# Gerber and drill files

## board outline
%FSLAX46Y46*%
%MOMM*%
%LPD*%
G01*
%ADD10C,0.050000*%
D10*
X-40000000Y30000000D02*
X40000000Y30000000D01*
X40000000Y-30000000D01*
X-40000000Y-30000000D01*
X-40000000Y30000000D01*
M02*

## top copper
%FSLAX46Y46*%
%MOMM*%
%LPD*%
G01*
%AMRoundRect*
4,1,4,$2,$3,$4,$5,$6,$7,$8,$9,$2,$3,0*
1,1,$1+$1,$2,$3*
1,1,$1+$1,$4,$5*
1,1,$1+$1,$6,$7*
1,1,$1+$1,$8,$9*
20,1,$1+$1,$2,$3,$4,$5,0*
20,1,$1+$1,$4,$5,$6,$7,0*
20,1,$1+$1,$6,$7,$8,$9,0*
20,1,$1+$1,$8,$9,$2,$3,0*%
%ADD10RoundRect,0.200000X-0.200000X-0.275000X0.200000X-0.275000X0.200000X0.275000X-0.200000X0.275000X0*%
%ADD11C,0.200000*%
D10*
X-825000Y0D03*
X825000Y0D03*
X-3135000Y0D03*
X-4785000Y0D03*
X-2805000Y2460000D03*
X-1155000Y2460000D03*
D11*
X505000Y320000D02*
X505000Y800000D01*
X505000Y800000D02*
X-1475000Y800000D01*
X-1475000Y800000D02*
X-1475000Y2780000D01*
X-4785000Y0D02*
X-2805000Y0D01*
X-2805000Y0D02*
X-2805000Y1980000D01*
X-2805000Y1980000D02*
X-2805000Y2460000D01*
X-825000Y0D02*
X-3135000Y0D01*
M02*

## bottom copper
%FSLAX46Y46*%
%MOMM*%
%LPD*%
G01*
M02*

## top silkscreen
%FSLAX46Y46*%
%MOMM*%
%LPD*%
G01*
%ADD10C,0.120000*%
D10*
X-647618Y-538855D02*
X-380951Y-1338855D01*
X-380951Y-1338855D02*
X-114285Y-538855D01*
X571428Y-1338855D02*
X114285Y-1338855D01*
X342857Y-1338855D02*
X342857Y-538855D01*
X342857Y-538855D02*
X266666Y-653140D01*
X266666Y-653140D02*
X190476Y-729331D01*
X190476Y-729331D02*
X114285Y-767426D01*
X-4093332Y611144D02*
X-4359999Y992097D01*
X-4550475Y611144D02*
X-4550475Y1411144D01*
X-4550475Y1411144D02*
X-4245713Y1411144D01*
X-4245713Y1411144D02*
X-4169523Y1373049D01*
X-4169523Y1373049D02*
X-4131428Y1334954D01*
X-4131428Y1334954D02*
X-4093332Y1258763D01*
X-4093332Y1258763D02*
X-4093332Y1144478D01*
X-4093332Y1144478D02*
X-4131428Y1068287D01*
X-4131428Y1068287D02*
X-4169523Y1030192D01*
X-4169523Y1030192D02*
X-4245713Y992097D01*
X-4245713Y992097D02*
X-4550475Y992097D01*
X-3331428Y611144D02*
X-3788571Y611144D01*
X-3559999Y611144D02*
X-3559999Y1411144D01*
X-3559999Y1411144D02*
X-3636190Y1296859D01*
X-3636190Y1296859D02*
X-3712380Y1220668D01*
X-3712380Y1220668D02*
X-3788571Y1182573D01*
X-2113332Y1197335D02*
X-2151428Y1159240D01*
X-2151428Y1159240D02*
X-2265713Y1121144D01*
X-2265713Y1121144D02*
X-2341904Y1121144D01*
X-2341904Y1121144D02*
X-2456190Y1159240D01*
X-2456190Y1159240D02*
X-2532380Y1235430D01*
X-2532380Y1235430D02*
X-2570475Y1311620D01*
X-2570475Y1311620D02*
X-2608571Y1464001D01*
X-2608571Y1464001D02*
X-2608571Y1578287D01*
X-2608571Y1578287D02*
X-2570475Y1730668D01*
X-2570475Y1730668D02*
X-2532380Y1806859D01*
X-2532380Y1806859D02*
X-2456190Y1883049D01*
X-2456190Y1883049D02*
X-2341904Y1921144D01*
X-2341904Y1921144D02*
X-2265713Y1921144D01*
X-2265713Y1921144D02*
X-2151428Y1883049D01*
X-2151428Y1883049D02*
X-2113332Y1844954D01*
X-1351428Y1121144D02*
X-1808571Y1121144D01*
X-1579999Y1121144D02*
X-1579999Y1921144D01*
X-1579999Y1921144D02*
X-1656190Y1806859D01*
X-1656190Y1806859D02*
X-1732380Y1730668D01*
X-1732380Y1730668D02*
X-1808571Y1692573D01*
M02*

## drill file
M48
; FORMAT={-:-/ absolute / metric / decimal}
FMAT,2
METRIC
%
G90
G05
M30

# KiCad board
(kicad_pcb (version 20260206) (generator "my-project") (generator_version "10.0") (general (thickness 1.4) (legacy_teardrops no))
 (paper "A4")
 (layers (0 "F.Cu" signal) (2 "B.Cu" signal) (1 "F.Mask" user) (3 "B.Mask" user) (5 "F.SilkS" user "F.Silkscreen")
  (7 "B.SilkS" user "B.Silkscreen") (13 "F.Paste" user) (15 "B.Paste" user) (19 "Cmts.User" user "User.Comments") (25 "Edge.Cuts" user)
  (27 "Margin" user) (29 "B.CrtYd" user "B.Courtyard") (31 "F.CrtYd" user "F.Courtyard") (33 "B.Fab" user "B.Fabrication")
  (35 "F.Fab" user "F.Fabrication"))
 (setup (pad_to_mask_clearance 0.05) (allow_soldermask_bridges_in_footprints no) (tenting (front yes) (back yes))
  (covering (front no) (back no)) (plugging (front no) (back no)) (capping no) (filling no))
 (gr_rect (start -40.0000 -30.0000) (end 40.0000 30.0000) (stroke (width 0.05) (type solid)) (fill none) (layer "Edge.Cuts"))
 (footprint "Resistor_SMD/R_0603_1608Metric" (layer "F.Cu") (at 0.0000 0.0000 0)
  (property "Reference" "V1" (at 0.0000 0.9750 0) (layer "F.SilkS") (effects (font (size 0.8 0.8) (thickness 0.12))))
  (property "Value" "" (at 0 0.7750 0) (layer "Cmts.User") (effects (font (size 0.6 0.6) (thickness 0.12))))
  (pad 1 smd roundrect (at -0.8250 0.0000) (size 0.8000 0.9500) (layers "F.Cu" "F.Mask") (roundrect_rratio 0.25) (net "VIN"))
  (pad 2 smd roundrect (at 0.8250 0.0000) (size 0.8000 0.9500) (layers "F.Cu" "F.Mask") (roundrect_rratio 0.25) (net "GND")))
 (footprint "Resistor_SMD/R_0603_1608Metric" (layer "F.Cu") (at -3.9600 0.0000 180)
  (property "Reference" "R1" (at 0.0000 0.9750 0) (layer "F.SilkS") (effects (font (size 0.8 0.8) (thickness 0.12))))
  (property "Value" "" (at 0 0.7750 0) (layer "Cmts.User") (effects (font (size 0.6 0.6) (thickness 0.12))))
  (pad 1 smd roundrect (at -0.8250 0.0000) (size 0.8000 0.9500) (layers "F.Cu" "F.Mask") (roundrect_rratio 0.25) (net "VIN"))
  (pad 2 smd roundrect (at 0.8250 -0.0000) (size 0.8000 0.9500) (layers "F.Cu" "F.Mask") (roundrect_rratio 0.25) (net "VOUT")))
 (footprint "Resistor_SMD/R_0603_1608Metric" (layer "F.Cu") (at -1.9800 -2.4600 0)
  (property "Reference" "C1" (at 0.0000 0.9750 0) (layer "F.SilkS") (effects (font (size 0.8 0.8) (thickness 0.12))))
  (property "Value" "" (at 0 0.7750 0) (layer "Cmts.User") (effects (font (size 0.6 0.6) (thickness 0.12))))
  (pad 1 smd roundrect (at -0.8250 0.0000) (size 0.8000 0.9500) (layers "F.Cu" "F.Mask") (roundrect_rratio 0.25) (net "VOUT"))
  (pad 2 smd roundrect (at 0.8250 0.0000) (size 0.8000 0.9500) (layers "F.Cu" "F.Mask") (roundrect_rratio 0.25) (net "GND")))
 (segment (start 0.5050 -0.3200) (end 0.5050 -0.8000) (width 0.2) (layer "F.Cu") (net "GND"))
 (segment (start 0.5050 -0.8000) (end -1.4750 -0.8000) (width 0.2) (layer "F.Cu") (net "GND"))
 (segment (start -1.4750 -0.8000) (end -1.4750 -2.7800) (width 0.2) (layer "F.Cu") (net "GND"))
 (segment (start -4.7850 0.0000) (end -2.8050 0.0000) (width 0.2) (layer "F.Cu") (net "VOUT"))
 (segment (start -2.8050 0.0000) (end -2.8050 -1.9800) (width 0.2) (layer "F.Cu") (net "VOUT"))
 (segment (start -2.8050 -1.9800) (end -2.8050 -2.4600) (width 0.2) (layer "F.Cu") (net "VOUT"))
 (segment (start -0.8250 0.0000) (end -3.1350 0.0000) (width 0.2) (layer "F.Cu") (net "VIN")))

